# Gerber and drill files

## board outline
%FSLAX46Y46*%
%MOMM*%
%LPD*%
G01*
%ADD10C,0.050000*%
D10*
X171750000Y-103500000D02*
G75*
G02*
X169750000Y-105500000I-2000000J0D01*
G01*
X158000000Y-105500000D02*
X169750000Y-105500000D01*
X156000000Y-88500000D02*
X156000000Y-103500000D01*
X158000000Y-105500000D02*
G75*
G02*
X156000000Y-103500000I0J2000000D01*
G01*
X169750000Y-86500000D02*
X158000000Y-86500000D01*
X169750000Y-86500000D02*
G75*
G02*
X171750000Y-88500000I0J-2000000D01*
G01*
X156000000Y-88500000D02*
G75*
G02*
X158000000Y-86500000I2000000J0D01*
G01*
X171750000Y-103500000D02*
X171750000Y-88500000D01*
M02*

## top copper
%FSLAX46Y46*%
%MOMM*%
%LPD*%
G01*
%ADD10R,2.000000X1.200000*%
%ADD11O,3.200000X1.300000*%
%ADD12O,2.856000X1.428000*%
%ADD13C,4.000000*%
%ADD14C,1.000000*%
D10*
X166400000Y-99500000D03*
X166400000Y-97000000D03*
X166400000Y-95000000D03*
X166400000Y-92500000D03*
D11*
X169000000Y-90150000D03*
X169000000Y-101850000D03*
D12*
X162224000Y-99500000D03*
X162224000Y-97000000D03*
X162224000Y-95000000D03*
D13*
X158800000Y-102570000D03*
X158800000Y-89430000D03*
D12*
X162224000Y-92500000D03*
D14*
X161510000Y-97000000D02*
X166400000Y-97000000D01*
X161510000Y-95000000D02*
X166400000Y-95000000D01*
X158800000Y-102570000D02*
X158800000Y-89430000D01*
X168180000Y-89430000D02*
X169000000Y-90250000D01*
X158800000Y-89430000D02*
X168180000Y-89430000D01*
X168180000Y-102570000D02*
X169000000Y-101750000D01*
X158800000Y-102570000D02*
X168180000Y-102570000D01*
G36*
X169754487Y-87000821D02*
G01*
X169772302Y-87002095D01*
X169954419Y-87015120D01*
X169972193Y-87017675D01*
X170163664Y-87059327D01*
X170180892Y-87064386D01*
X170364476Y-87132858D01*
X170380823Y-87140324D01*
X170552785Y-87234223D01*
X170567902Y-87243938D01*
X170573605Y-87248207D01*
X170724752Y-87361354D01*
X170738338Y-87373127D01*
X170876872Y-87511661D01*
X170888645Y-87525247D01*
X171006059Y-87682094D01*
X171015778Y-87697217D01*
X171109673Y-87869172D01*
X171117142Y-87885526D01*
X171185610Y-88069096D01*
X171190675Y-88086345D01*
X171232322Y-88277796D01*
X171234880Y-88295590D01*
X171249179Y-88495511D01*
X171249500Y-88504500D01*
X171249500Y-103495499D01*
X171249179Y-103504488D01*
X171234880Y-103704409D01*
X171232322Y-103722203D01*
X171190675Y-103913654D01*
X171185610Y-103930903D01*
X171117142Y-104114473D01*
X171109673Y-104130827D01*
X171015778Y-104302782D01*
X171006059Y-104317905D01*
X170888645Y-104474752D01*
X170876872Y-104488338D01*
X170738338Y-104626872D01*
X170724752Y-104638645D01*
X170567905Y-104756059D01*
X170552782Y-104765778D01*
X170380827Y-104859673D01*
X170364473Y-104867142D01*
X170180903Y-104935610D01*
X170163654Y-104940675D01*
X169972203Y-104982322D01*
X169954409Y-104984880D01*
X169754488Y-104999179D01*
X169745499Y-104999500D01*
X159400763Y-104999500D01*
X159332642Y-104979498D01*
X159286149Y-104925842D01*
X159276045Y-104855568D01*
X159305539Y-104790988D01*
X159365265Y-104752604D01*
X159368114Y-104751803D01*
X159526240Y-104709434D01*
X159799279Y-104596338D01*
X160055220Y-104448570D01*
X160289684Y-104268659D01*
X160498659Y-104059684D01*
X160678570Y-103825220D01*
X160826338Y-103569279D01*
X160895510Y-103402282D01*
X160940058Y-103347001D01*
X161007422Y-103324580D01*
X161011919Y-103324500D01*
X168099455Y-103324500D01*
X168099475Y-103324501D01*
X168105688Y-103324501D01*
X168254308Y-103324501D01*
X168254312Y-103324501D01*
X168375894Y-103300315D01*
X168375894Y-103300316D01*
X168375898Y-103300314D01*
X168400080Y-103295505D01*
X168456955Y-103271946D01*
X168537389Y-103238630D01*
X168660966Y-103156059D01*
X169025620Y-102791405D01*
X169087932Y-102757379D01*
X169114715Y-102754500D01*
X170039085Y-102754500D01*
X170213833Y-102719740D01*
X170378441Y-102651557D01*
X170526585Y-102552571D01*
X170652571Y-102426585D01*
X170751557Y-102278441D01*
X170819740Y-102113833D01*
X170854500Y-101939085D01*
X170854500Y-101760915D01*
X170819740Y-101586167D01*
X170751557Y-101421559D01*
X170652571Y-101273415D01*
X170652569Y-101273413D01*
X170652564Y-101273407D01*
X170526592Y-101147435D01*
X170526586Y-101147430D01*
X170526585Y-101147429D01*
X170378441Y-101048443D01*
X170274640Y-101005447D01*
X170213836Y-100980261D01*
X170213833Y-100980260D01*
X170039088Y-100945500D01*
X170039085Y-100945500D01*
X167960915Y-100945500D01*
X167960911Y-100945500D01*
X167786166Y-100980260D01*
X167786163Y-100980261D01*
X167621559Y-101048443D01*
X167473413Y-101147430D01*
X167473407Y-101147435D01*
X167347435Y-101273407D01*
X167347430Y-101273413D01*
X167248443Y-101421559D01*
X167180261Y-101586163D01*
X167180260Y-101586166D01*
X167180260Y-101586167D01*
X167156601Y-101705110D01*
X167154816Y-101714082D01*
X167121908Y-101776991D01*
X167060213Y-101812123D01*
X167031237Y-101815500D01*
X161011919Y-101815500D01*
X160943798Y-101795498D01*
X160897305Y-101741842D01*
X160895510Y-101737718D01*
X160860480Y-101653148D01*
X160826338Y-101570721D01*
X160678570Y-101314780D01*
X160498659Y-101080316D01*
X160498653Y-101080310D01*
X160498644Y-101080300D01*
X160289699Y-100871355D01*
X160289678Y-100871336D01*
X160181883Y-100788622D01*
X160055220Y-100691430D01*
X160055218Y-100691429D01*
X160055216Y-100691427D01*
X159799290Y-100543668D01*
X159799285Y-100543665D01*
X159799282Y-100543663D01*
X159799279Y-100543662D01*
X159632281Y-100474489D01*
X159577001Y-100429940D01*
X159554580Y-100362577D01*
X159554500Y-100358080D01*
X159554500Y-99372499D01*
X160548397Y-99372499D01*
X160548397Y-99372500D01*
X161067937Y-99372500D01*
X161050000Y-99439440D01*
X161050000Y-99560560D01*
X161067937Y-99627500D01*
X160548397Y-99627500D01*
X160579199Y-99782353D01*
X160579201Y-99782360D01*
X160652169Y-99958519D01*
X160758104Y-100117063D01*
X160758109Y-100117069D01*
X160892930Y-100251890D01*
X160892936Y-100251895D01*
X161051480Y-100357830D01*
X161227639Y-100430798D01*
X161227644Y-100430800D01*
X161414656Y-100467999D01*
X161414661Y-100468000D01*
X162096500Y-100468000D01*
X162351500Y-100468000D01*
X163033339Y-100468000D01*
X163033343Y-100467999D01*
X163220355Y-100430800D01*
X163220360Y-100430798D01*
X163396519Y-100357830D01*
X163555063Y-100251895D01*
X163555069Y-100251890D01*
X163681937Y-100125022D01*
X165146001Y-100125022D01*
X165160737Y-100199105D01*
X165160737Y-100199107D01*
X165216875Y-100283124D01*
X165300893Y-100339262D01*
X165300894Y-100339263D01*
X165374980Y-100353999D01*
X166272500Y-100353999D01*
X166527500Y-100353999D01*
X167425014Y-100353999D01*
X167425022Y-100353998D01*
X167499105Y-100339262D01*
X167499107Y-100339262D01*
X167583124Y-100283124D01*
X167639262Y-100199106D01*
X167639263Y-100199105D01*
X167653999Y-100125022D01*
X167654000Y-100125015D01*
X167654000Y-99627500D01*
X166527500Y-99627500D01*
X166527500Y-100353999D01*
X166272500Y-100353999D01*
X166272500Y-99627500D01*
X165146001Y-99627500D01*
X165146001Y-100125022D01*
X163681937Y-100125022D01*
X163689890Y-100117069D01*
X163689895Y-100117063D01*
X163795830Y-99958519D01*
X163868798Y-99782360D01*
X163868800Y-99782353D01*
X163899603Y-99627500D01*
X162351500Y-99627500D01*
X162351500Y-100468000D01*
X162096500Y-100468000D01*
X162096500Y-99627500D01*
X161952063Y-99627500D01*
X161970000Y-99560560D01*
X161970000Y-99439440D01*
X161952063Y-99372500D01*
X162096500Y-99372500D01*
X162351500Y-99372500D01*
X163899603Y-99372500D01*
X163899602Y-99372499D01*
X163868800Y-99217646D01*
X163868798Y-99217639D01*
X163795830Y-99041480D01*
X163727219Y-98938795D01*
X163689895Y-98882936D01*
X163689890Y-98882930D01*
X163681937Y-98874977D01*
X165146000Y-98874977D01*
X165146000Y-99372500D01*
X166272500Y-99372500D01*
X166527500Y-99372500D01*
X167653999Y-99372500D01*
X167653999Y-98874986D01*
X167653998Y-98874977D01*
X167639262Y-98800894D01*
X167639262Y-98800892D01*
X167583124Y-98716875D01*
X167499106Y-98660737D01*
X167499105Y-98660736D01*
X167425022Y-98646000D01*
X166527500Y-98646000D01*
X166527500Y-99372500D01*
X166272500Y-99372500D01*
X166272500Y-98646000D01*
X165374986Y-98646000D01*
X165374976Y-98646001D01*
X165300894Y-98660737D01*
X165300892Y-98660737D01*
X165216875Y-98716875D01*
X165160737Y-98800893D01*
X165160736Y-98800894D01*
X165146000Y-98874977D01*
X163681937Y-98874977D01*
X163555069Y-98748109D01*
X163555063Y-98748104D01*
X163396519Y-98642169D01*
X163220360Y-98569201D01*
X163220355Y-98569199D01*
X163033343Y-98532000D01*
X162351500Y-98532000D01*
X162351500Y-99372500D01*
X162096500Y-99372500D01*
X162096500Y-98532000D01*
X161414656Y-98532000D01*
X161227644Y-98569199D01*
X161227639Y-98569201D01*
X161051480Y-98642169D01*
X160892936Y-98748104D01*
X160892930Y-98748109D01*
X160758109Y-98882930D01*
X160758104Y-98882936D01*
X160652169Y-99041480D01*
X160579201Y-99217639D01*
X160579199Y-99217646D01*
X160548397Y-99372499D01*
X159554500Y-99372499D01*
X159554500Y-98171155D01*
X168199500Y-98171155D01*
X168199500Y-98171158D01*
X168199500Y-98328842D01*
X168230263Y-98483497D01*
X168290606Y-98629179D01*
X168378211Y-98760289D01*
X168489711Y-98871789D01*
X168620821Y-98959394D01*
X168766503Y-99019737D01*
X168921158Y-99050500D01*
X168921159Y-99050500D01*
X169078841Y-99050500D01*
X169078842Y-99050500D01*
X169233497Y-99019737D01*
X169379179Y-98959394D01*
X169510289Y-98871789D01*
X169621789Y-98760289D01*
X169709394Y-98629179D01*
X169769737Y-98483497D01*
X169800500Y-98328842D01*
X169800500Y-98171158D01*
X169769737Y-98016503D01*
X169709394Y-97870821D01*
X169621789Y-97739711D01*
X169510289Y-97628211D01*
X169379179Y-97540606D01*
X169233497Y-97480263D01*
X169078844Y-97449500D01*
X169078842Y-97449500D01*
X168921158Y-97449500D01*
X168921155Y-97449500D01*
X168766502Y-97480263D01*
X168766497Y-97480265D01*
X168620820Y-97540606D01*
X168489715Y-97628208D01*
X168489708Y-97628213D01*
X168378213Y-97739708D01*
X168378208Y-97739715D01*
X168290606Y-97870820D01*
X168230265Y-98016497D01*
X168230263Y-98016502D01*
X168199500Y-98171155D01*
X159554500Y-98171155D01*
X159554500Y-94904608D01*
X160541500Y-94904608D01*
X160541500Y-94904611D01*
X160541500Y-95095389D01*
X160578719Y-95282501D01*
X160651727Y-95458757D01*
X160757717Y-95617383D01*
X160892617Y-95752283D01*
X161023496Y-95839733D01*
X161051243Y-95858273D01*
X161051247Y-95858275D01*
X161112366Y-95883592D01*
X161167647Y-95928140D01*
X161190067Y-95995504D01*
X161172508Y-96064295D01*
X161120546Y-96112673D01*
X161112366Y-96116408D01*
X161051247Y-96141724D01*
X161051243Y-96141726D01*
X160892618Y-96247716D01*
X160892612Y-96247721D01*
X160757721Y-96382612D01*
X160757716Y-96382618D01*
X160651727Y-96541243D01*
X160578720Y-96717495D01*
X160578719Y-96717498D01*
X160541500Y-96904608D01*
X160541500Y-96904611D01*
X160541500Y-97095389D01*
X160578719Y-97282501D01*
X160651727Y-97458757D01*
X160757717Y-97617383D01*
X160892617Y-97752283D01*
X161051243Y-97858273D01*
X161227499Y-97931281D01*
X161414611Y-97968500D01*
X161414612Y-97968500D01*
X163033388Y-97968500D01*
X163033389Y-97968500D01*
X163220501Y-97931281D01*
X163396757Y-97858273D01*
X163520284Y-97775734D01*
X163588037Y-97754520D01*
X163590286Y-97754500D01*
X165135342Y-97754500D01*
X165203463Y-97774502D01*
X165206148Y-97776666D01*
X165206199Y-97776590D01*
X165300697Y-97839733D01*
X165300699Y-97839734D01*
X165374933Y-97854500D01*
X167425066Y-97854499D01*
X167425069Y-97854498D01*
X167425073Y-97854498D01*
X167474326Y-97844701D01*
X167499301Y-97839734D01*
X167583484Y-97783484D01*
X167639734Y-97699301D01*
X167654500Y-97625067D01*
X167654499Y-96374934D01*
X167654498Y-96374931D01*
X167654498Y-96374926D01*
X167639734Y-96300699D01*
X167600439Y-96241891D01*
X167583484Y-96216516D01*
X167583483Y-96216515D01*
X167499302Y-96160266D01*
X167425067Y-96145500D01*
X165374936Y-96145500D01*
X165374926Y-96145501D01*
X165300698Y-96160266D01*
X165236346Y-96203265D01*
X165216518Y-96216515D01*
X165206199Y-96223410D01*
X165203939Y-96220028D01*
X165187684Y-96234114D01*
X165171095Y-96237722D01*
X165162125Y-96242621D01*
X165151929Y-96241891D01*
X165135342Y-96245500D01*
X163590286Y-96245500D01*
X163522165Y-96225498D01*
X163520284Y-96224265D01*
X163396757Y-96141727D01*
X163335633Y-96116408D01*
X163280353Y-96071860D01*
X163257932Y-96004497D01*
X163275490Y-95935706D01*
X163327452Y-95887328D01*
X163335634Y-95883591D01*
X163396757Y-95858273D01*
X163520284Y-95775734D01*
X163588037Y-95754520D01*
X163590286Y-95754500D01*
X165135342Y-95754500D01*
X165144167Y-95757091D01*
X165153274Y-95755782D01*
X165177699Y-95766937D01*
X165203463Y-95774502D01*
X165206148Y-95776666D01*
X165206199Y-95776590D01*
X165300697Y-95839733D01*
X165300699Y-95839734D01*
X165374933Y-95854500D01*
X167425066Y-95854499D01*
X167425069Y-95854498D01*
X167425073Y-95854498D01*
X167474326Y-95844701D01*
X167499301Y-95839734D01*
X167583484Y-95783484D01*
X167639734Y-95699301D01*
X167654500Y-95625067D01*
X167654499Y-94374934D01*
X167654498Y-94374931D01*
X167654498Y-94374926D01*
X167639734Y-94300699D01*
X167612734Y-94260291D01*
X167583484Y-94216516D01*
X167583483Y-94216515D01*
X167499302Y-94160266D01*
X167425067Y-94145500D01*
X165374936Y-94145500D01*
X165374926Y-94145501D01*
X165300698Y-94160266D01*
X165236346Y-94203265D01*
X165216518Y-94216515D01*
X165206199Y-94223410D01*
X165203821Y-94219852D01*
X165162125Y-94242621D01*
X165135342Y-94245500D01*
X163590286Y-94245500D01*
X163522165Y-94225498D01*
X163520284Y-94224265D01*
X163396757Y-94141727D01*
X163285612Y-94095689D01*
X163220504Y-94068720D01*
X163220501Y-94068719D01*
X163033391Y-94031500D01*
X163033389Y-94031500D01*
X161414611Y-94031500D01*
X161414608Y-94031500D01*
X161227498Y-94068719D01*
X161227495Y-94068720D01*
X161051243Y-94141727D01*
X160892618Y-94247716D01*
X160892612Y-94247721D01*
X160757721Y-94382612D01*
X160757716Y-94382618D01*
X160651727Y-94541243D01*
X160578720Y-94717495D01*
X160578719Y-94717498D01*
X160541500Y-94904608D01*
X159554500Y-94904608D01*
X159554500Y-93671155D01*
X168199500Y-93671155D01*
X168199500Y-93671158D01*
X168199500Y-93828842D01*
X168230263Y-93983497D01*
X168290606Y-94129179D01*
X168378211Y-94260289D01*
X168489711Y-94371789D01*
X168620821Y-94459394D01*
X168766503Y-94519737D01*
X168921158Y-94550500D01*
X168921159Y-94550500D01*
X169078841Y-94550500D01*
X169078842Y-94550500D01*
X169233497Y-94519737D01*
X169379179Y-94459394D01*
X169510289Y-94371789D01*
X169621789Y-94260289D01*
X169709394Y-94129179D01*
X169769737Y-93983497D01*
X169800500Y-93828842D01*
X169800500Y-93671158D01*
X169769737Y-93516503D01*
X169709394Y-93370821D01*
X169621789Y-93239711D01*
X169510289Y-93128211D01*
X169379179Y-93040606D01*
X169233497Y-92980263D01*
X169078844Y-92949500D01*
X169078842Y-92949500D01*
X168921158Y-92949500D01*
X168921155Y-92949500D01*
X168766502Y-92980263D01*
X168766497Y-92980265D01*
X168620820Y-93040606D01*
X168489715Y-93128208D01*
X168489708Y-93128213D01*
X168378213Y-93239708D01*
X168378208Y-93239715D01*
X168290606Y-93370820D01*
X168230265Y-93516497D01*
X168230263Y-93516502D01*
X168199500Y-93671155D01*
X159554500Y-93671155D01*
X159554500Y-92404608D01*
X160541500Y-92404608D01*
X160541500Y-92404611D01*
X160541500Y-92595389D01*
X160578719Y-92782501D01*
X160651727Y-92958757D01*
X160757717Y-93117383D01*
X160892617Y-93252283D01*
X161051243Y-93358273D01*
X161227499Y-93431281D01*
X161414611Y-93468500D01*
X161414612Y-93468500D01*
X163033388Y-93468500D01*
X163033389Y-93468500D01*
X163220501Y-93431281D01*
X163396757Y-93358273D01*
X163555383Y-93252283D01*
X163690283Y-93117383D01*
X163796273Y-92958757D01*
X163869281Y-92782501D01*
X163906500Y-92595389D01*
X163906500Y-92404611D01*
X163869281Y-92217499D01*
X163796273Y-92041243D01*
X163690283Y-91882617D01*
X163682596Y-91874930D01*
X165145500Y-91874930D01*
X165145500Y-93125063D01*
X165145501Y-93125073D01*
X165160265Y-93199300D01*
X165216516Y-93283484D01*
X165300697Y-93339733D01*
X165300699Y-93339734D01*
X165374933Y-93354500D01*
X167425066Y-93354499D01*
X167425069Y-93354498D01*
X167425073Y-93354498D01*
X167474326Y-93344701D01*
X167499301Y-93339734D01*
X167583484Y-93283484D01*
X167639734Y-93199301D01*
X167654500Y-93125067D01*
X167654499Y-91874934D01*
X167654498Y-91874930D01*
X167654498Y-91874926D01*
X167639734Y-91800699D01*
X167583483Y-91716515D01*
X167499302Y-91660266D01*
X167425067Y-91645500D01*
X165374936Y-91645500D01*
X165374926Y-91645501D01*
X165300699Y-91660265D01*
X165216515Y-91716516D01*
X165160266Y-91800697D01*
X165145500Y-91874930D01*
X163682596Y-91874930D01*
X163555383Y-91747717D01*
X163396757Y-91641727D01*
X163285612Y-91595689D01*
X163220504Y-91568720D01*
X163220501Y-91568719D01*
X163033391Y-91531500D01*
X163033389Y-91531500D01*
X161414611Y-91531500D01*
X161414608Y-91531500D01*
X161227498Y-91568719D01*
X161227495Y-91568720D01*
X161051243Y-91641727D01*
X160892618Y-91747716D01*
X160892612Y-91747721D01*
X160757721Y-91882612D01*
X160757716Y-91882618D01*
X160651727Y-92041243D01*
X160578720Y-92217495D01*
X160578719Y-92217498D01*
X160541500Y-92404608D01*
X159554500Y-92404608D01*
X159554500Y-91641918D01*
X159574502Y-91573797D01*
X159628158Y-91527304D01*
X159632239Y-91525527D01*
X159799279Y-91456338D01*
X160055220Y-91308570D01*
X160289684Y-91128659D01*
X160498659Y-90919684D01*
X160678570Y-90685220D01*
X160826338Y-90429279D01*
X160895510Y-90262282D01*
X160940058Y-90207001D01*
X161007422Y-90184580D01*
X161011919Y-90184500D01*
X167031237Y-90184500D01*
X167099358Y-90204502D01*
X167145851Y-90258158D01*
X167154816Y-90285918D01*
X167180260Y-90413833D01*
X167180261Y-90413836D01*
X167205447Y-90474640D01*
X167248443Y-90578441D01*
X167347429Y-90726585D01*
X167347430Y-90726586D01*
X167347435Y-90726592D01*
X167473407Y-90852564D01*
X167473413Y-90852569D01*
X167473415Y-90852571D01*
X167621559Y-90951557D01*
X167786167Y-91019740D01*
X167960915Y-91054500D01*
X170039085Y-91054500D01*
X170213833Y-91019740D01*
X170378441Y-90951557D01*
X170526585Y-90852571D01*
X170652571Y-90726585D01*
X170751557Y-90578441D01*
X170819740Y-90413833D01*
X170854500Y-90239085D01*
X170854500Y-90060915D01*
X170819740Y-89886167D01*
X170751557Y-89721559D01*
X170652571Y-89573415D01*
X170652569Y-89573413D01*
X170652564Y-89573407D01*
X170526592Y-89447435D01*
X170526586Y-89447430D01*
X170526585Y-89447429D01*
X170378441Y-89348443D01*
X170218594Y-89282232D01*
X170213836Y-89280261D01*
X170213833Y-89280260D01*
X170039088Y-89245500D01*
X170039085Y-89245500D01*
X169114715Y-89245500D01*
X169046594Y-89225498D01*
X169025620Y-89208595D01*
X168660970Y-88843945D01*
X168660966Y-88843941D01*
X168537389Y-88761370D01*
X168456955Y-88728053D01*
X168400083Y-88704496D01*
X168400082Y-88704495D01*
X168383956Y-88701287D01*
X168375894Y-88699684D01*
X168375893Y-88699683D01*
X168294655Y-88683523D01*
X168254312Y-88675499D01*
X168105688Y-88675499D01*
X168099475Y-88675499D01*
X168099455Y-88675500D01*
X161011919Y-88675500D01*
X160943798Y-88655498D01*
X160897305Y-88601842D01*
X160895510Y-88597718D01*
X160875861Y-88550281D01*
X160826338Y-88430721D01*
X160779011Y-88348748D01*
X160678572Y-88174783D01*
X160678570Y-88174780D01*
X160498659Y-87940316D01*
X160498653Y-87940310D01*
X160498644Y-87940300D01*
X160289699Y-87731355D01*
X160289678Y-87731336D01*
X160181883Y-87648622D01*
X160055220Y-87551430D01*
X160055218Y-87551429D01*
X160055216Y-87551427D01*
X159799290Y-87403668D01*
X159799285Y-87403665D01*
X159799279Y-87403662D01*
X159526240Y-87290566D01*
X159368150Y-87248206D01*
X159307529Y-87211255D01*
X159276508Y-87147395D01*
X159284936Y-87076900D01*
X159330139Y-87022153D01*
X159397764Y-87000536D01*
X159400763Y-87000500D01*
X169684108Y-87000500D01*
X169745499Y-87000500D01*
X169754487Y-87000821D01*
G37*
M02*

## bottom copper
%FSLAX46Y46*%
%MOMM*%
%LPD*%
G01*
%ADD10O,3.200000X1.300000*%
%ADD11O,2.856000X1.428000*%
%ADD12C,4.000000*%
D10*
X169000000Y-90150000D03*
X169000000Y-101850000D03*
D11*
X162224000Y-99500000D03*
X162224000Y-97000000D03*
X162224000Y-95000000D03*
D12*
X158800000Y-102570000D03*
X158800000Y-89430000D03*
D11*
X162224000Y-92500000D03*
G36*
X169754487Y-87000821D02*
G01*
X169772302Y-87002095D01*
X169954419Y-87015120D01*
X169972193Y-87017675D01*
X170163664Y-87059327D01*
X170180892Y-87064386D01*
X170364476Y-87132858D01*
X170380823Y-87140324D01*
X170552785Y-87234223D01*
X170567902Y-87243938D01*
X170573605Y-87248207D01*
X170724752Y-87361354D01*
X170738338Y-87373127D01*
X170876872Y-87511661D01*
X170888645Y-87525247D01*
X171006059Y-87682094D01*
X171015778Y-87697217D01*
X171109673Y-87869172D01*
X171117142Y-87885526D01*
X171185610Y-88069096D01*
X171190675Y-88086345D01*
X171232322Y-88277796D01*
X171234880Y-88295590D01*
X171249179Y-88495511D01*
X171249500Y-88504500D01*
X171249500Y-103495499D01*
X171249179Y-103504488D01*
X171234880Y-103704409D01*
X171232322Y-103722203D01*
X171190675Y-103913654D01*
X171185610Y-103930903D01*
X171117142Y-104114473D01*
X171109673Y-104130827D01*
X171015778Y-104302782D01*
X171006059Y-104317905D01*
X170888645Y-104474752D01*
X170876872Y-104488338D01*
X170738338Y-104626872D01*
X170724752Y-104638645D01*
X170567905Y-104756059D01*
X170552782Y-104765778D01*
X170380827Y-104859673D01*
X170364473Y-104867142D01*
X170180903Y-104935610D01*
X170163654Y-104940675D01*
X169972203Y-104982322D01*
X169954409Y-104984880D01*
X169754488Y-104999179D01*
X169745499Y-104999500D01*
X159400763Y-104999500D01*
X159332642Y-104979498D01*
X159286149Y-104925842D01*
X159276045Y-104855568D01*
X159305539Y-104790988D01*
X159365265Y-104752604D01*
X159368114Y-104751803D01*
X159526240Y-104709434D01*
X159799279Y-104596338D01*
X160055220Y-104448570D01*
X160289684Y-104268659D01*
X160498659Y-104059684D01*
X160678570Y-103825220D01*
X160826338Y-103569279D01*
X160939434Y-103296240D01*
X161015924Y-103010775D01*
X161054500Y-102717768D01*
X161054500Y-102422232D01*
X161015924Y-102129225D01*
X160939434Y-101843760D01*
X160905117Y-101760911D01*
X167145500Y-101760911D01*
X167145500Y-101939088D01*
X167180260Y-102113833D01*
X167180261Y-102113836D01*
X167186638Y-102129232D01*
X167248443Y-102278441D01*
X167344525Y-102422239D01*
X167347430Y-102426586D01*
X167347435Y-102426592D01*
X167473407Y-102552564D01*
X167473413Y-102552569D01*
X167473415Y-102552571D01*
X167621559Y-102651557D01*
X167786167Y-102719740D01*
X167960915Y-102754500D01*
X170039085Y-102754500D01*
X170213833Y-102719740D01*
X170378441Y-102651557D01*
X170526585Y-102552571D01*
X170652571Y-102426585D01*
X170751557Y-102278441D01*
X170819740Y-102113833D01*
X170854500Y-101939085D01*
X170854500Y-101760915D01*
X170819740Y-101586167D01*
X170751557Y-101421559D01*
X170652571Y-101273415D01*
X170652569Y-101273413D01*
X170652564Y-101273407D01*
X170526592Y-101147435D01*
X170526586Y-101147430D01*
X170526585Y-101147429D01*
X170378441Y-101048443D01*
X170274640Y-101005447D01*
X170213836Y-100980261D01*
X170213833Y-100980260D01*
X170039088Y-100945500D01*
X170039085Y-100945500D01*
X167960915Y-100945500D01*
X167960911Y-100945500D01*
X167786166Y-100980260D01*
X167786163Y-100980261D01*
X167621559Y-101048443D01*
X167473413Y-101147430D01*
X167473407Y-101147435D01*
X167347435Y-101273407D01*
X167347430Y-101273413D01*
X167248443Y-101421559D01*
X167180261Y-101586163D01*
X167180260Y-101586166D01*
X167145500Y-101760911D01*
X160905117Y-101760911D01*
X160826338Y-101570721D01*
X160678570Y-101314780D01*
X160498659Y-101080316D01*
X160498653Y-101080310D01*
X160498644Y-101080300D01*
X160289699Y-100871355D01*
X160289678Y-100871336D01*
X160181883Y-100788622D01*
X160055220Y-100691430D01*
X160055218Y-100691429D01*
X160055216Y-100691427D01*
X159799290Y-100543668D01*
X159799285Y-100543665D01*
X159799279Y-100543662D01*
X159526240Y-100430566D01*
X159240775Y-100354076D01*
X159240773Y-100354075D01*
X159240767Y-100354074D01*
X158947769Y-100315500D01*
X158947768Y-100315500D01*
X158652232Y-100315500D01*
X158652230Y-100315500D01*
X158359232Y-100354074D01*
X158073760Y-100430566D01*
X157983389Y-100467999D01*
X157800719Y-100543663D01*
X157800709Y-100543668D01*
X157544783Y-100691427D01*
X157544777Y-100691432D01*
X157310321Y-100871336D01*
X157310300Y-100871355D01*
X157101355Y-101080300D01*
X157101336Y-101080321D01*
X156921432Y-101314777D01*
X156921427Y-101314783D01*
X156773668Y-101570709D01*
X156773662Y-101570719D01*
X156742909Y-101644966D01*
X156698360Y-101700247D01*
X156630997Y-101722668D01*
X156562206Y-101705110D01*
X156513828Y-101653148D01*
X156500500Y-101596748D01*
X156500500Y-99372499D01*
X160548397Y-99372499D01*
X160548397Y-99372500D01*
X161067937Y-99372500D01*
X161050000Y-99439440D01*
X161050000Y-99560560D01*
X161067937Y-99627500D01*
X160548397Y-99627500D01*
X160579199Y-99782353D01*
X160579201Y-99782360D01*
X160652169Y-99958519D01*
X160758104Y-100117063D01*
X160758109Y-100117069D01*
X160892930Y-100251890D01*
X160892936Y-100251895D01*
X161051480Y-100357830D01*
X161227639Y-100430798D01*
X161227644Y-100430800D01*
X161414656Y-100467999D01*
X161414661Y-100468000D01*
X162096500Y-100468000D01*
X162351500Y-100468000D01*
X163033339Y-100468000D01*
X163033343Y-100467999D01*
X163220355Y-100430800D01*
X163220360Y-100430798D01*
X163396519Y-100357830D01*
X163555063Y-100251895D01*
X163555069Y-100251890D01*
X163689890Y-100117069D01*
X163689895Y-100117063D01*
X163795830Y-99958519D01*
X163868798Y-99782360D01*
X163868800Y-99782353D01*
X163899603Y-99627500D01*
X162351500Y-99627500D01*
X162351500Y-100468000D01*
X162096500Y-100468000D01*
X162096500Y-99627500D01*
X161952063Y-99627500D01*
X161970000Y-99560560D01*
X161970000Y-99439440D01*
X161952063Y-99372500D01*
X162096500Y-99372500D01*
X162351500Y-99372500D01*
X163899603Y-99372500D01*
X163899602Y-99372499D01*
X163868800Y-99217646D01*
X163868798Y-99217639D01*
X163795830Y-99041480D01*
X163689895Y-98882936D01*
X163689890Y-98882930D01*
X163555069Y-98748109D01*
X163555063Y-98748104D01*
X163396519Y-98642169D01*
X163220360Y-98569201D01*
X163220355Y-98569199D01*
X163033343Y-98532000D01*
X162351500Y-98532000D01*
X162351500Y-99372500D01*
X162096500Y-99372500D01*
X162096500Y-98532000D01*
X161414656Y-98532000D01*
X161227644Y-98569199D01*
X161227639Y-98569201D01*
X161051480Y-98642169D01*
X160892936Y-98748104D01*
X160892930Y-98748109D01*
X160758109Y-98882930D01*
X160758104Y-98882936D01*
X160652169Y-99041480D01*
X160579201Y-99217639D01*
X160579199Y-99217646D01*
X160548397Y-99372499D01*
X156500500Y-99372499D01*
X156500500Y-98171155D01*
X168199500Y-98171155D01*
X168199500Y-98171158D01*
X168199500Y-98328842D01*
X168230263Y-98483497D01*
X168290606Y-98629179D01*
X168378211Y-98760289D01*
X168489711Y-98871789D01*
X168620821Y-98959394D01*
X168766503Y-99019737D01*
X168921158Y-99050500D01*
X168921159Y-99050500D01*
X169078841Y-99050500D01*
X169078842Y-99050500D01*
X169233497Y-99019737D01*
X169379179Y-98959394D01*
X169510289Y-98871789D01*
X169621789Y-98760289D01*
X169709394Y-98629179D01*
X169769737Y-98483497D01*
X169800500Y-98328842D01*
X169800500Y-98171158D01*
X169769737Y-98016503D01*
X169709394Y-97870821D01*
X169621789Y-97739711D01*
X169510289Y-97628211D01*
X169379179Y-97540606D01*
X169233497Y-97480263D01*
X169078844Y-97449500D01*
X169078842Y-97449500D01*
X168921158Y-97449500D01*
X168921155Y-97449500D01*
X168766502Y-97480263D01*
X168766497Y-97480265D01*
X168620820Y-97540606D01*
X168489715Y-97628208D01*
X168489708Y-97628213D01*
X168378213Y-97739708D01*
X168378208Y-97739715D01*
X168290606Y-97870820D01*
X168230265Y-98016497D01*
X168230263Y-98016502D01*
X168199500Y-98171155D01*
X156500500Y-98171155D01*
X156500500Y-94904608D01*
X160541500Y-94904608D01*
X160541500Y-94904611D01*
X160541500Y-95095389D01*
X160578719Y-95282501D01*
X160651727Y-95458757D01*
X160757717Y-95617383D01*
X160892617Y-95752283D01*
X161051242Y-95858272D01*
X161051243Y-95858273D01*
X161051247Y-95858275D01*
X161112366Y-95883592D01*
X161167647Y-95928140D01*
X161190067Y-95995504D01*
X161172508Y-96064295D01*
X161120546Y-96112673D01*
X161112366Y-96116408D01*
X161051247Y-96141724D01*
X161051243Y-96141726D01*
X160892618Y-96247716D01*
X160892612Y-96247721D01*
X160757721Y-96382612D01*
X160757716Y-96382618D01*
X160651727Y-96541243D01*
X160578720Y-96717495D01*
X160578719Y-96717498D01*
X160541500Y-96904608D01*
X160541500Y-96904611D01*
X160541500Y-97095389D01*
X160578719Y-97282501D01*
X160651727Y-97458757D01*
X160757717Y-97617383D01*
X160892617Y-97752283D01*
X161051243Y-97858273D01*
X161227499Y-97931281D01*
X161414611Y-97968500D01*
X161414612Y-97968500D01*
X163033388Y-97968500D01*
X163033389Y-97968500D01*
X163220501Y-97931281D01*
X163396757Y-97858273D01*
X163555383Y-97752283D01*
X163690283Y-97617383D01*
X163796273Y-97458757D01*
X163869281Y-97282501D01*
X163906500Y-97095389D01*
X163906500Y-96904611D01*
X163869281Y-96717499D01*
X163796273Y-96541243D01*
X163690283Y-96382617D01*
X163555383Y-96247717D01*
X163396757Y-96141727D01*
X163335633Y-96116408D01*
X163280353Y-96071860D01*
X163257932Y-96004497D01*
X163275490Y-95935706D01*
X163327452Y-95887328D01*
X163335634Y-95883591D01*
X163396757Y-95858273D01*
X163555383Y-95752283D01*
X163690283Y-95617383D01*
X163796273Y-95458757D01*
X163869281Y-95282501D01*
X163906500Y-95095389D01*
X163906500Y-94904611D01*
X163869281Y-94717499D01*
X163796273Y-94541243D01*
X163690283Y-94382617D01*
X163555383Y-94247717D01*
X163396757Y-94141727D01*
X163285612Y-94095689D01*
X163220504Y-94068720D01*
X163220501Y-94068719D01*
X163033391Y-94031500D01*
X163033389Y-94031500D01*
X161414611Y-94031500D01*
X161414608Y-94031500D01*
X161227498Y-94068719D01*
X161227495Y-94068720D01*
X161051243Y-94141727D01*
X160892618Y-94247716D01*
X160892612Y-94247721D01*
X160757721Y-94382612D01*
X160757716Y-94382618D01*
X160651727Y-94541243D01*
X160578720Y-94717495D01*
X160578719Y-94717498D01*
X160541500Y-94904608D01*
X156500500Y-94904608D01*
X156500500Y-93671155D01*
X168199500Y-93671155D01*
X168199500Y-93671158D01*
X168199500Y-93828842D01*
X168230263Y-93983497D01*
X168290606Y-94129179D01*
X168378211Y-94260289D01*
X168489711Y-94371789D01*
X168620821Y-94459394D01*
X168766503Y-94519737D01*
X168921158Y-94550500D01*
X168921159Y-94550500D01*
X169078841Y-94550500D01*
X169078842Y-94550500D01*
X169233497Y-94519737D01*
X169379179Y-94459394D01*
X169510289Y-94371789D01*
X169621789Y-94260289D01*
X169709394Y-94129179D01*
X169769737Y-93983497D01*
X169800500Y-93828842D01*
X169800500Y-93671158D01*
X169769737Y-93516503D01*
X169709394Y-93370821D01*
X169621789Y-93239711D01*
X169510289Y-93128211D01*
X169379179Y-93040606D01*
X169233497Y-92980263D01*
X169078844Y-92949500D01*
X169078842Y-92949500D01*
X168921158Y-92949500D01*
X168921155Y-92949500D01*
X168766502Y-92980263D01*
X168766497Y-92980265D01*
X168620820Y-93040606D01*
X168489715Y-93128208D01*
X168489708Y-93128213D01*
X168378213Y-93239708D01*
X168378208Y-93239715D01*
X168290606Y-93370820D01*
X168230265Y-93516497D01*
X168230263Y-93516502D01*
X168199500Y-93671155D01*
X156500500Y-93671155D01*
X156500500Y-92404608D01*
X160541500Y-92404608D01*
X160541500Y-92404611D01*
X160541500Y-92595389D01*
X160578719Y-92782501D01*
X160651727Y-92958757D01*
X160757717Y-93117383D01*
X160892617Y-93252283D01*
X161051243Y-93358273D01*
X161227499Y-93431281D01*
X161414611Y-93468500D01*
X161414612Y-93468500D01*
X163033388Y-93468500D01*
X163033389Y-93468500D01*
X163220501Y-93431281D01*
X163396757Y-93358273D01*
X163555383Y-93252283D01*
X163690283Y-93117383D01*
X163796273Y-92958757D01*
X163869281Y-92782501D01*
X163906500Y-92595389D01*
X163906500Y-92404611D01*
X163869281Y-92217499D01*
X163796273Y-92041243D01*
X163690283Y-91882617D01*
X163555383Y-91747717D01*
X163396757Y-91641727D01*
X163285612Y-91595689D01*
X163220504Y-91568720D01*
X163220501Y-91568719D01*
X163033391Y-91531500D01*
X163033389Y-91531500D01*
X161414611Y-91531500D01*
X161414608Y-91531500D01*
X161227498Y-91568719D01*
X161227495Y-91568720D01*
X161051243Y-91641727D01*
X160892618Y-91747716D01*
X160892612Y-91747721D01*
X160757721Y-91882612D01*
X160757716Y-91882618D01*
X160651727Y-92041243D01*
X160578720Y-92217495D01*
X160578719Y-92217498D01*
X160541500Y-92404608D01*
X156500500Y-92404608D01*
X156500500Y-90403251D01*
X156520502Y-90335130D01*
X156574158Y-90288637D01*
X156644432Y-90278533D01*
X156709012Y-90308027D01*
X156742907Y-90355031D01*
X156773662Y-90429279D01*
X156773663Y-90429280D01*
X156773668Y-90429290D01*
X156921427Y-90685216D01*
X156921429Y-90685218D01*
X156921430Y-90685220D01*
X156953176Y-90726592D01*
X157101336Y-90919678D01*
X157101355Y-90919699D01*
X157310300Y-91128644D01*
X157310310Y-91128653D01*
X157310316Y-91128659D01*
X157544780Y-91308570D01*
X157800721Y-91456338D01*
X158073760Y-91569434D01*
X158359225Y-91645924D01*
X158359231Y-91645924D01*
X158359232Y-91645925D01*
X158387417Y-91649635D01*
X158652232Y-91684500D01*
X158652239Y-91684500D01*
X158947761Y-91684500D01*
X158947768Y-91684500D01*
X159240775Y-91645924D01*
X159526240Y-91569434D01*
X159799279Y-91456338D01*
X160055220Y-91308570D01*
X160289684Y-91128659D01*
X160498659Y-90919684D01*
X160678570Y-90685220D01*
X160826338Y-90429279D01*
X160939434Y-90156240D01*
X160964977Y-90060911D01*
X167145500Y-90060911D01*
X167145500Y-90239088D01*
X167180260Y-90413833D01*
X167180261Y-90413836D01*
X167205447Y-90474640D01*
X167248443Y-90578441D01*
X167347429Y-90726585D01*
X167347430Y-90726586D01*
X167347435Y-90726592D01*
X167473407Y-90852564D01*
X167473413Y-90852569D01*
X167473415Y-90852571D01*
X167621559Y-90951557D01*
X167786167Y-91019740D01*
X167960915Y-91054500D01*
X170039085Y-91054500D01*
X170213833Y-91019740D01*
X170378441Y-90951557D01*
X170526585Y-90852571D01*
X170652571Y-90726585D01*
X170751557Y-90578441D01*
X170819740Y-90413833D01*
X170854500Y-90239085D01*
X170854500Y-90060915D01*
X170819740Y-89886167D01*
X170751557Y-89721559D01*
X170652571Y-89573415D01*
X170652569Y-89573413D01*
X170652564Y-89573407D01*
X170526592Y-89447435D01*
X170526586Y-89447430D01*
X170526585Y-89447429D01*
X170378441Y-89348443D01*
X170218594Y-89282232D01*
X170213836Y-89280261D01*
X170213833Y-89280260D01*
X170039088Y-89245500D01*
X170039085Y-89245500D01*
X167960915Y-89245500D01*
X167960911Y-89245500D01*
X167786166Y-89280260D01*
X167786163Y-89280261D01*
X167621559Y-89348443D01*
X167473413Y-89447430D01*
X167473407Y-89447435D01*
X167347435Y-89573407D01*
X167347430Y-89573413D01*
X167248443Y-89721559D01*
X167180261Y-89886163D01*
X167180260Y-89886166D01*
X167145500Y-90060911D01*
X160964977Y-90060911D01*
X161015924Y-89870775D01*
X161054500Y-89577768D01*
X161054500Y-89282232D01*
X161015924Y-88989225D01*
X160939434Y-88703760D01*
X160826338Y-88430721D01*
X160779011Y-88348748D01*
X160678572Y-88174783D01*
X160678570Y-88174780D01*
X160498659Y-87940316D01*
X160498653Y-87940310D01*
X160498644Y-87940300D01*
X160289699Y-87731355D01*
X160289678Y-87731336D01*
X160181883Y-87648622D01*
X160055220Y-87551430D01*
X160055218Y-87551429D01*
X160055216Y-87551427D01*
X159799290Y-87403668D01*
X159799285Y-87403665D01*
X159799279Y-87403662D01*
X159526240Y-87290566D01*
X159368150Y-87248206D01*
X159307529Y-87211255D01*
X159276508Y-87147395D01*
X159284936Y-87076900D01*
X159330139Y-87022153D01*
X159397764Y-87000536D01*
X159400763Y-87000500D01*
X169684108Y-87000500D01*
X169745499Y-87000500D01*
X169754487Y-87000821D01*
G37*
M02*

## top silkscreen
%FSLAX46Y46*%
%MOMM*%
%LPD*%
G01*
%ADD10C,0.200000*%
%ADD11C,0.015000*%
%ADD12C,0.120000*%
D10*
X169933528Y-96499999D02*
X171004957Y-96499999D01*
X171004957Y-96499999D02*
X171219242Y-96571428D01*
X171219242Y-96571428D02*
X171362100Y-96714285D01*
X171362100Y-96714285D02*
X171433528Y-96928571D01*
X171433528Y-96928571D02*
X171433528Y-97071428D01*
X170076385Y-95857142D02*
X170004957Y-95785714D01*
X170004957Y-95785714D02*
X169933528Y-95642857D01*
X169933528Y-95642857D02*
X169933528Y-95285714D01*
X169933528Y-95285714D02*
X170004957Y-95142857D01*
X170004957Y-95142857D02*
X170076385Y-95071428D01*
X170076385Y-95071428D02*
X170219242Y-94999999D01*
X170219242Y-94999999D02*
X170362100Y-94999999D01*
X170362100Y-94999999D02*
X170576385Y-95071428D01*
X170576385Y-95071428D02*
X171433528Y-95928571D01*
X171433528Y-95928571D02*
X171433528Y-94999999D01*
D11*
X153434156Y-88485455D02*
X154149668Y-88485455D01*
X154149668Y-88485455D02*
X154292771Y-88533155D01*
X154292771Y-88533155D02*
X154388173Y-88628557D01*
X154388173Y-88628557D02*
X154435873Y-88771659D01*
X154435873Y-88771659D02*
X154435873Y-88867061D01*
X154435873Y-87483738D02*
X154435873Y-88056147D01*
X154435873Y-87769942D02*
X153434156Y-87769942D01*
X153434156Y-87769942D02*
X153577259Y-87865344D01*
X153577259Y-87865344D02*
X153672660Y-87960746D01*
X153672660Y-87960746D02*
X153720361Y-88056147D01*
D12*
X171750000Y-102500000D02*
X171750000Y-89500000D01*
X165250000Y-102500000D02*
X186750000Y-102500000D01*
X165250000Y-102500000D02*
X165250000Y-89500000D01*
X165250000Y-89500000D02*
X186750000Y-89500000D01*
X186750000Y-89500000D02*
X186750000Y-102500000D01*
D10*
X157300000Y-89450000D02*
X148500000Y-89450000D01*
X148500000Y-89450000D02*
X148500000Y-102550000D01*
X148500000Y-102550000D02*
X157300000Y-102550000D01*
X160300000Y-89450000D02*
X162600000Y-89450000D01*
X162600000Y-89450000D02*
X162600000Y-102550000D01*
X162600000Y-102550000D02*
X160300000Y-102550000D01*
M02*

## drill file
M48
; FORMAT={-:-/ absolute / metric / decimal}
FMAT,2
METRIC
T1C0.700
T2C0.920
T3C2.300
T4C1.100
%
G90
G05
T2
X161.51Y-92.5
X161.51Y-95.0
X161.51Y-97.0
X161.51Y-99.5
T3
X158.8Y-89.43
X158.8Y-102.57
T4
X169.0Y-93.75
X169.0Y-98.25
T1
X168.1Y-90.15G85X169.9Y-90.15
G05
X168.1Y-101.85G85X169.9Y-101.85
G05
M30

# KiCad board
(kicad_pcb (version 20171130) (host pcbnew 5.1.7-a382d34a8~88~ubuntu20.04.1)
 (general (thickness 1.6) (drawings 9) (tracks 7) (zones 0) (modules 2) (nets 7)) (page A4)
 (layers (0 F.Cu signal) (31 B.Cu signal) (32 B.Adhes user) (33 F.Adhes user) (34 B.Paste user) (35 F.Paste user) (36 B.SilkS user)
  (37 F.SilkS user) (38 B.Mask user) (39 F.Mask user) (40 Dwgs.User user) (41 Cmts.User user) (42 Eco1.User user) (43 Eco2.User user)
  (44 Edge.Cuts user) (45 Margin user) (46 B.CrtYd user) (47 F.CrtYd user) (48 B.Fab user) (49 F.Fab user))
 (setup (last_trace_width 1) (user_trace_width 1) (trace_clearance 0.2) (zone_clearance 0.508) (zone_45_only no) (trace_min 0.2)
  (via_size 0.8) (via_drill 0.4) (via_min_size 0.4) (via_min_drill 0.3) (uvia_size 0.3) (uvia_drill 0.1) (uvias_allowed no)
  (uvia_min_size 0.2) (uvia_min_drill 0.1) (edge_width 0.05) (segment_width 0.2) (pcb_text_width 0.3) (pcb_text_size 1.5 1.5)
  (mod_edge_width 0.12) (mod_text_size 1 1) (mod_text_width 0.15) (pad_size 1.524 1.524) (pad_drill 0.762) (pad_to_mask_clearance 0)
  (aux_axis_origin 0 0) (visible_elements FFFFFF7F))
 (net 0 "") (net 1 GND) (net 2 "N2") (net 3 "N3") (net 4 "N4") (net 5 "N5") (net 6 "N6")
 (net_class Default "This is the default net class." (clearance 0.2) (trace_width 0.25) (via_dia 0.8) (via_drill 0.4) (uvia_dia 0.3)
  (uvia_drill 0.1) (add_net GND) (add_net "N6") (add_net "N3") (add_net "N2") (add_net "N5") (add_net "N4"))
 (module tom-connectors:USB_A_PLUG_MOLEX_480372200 (layer F.Cu) (at 169 96 90)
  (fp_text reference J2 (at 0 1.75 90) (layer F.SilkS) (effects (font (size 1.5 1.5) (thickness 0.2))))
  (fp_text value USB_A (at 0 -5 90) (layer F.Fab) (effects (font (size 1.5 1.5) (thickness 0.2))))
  (fp_line (start -6.5 2.75) (end 6.5 2.75) (layer F.SilkS) (width 0.12))
  (fp_line (start -6.5 -3.75) (end -6.5 17.75) (layer F.SilkS) (width 0.12))
  (fp_line (start -6.5 -3.75) (end 6.5 -3.75) (layer F.SilkS) (width 0.12))
  (fp_line (start 6.5 -3.75) (end 6.5 17.75) (layer F.SilkS) (width 0.12))
  (fp_line (start 6.5 17.75) (end -6.5 17.75) (layer F.SilkS) (width 0.12))
  (pad "" np_thru_hole circle (at 2.25 0 90) (size 1.1 1.1) (drill 1.1) (layers *.Cu *.Mask))
  (pad "" np_thru_hole circle (at -2.25 0 90) (size 1.1 1.1) (drill 1.1) (layers *.Cu *.Mask))
  (pad 4 smd rect (at -3.5 -2.6 90) (size 1.2 2) (layers F.Cu F.Paste F.Mask) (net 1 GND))
  (pad 3 smd rect (at -1 -2.6 90) (size 1.2 2) (layers F.Cu F.Paste F.Mask) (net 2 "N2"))
  (pad 2 smd rect (at 1 -2.6 90) (size 1.2 2) (layers F.Cu F.Paste F.Mask) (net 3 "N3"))
  (pad 1 smd rect (at 3.5 -2.6 90) (size 1.2 2) (layers F.Cu F.Paste F.Mask) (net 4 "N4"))
  (pad 5 thru_hole oval (at 5.85 0 90) (size 1.3 3.2) (drill oval 0.7 2.5) (layers *.Cu *.Mask) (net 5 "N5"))
  (pad 5 thru_hole oval (at -5.85 0 90) (size 1.3 3.2) (drill oval 0.7 2.5) (layers *.Cu *.Mask) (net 5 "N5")))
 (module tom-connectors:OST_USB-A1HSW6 (layer F.Cu) (at 155 96 270)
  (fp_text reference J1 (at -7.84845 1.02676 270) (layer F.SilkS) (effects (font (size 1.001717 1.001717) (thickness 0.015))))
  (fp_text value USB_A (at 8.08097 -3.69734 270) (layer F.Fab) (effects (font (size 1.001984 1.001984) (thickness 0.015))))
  (fp_line (start -6.55 -2.3) (end -6.55 6.5) (layer F.SilkS) (width 0.2))
  (fp_line (start -6.55 6.5) (end 6.55 6.5) (layer F.SilkS) (width 0.2))
  (fp_line (start 6.55 6.5) (end 6.55 -2.3) (layer F.SilkS) (width 0.2))
  (fp_line (start -6.55 -5.3) (end -6.55 -7.6) (layer F.SilkS) (width 0.2))
  (fp_line (start -6.55 -7.6) (end 6.55 -7.6) (layer F.SilkS) (width 0.2))
  (fp_line (start 6.55 -7.6) (end 6.55 -5.3) (layer F.SilkS) (width 0.2))
  (pad 4 thru_hole oval (at 3.5 -6.51 270) (size 1.428 2.856) (drill oval 0.92 (offset 0 -0.714)) (layers *.Cu *.Mask) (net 1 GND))
  (pad 3 thru_hole oval (at 1 -6.51 270) (size 1.428 2.856) (drill oval 0.92 (offset 0 -0.714)) (layers *.Cu *.Mask) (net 2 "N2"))
  (pad 2 thru_hole oval (at -1 -6.51 270) (size 1.428 2.856) (drill oval 0.92 (offset 0 -0.714)) (layers *.Cu *.Mask) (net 3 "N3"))
  (pad 5 thru_hole circle (at 6.57 -3.8 270) (size 4 4) (drill 2.3) (layers *.Cu *.Mask) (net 5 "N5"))
  (pad 5 thru_hole circle (at -6.57 -3.8 270) (size 4 4) (drill 2.3) (layers *.Cu *.Mask) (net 5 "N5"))
  (pad 1 thru_hole oval (at -3.5 -6.51 270) (size 1.428 2.856) (drill oval 0.92 (offset 0 -0.714)) (layers *.Cu *.Mask) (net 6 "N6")))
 (gr_arc (start 169.75 103.5) (end 169.75 105.5) (angle -90) (layer Edge.Cuts) (width 0.05))
 (gr_line (start 158 105.5) (end 169.75 105.5) (layer Edge.Cuts) (width 0.05))
 (gr_line (start 156 88.5) (end 156 103.5) (layer Edge.Cuts) (width 0.05))
 (gr_arc (start 158 103.5) (end 156 103.5) (angle -90) (layer Edge.Cuts) (width 0.05))
 (gr_line (start 169.75 86.5) (end 158 86.5) (layer Edge.Cuts) (width 0.05))
 (gr_arc (start 169.75 88.5) (end 171.75 88.5) (angle -90) (layer Edge.Cuts) (width 0.05))
 (gr_arc (start 158 88.5) (end 158 86.5) (angle -90) (layer Edge.Cuts) (width 0.05))
 (gr_line (start 171.75 103.5) (end 171.75 88.5) (layer Edge.Cuts) (width 0.05))
 (segment (start 161.51 97) (end 166.4 97) (width 1) (layer F.Cu) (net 2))
 (segment (start 161.51 95) (end 166.4 95) (width 1) (layer F.Cu) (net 3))
 (segment (start 158.8 102.57) (end 158.8 89.43) (width 1) (layer F.Cu) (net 5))
 (segment (start 168.18 89.43) (end 169 90.25) (width 1) (layer F.Cu) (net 5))
 (segment (start 158.8 89.43) (end 168.18 89.43) (width 1) (layer F.Cu) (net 5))
 (segment (start 168.18 102.57) (end 169 101.75) (width 1) (layer F.Cu) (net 5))
 (segment (start 158.8 102.57) (end 168.18 102.57) (width 1) (layer F.Cu) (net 5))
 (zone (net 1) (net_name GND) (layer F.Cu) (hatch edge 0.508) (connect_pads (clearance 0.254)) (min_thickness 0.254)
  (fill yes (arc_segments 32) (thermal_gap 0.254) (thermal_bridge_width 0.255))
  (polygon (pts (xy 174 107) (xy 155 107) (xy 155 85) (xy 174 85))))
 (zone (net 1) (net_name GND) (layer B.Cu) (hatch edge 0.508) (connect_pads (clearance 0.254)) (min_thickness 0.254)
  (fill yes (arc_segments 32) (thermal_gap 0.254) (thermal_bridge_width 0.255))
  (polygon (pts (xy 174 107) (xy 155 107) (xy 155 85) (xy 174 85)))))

